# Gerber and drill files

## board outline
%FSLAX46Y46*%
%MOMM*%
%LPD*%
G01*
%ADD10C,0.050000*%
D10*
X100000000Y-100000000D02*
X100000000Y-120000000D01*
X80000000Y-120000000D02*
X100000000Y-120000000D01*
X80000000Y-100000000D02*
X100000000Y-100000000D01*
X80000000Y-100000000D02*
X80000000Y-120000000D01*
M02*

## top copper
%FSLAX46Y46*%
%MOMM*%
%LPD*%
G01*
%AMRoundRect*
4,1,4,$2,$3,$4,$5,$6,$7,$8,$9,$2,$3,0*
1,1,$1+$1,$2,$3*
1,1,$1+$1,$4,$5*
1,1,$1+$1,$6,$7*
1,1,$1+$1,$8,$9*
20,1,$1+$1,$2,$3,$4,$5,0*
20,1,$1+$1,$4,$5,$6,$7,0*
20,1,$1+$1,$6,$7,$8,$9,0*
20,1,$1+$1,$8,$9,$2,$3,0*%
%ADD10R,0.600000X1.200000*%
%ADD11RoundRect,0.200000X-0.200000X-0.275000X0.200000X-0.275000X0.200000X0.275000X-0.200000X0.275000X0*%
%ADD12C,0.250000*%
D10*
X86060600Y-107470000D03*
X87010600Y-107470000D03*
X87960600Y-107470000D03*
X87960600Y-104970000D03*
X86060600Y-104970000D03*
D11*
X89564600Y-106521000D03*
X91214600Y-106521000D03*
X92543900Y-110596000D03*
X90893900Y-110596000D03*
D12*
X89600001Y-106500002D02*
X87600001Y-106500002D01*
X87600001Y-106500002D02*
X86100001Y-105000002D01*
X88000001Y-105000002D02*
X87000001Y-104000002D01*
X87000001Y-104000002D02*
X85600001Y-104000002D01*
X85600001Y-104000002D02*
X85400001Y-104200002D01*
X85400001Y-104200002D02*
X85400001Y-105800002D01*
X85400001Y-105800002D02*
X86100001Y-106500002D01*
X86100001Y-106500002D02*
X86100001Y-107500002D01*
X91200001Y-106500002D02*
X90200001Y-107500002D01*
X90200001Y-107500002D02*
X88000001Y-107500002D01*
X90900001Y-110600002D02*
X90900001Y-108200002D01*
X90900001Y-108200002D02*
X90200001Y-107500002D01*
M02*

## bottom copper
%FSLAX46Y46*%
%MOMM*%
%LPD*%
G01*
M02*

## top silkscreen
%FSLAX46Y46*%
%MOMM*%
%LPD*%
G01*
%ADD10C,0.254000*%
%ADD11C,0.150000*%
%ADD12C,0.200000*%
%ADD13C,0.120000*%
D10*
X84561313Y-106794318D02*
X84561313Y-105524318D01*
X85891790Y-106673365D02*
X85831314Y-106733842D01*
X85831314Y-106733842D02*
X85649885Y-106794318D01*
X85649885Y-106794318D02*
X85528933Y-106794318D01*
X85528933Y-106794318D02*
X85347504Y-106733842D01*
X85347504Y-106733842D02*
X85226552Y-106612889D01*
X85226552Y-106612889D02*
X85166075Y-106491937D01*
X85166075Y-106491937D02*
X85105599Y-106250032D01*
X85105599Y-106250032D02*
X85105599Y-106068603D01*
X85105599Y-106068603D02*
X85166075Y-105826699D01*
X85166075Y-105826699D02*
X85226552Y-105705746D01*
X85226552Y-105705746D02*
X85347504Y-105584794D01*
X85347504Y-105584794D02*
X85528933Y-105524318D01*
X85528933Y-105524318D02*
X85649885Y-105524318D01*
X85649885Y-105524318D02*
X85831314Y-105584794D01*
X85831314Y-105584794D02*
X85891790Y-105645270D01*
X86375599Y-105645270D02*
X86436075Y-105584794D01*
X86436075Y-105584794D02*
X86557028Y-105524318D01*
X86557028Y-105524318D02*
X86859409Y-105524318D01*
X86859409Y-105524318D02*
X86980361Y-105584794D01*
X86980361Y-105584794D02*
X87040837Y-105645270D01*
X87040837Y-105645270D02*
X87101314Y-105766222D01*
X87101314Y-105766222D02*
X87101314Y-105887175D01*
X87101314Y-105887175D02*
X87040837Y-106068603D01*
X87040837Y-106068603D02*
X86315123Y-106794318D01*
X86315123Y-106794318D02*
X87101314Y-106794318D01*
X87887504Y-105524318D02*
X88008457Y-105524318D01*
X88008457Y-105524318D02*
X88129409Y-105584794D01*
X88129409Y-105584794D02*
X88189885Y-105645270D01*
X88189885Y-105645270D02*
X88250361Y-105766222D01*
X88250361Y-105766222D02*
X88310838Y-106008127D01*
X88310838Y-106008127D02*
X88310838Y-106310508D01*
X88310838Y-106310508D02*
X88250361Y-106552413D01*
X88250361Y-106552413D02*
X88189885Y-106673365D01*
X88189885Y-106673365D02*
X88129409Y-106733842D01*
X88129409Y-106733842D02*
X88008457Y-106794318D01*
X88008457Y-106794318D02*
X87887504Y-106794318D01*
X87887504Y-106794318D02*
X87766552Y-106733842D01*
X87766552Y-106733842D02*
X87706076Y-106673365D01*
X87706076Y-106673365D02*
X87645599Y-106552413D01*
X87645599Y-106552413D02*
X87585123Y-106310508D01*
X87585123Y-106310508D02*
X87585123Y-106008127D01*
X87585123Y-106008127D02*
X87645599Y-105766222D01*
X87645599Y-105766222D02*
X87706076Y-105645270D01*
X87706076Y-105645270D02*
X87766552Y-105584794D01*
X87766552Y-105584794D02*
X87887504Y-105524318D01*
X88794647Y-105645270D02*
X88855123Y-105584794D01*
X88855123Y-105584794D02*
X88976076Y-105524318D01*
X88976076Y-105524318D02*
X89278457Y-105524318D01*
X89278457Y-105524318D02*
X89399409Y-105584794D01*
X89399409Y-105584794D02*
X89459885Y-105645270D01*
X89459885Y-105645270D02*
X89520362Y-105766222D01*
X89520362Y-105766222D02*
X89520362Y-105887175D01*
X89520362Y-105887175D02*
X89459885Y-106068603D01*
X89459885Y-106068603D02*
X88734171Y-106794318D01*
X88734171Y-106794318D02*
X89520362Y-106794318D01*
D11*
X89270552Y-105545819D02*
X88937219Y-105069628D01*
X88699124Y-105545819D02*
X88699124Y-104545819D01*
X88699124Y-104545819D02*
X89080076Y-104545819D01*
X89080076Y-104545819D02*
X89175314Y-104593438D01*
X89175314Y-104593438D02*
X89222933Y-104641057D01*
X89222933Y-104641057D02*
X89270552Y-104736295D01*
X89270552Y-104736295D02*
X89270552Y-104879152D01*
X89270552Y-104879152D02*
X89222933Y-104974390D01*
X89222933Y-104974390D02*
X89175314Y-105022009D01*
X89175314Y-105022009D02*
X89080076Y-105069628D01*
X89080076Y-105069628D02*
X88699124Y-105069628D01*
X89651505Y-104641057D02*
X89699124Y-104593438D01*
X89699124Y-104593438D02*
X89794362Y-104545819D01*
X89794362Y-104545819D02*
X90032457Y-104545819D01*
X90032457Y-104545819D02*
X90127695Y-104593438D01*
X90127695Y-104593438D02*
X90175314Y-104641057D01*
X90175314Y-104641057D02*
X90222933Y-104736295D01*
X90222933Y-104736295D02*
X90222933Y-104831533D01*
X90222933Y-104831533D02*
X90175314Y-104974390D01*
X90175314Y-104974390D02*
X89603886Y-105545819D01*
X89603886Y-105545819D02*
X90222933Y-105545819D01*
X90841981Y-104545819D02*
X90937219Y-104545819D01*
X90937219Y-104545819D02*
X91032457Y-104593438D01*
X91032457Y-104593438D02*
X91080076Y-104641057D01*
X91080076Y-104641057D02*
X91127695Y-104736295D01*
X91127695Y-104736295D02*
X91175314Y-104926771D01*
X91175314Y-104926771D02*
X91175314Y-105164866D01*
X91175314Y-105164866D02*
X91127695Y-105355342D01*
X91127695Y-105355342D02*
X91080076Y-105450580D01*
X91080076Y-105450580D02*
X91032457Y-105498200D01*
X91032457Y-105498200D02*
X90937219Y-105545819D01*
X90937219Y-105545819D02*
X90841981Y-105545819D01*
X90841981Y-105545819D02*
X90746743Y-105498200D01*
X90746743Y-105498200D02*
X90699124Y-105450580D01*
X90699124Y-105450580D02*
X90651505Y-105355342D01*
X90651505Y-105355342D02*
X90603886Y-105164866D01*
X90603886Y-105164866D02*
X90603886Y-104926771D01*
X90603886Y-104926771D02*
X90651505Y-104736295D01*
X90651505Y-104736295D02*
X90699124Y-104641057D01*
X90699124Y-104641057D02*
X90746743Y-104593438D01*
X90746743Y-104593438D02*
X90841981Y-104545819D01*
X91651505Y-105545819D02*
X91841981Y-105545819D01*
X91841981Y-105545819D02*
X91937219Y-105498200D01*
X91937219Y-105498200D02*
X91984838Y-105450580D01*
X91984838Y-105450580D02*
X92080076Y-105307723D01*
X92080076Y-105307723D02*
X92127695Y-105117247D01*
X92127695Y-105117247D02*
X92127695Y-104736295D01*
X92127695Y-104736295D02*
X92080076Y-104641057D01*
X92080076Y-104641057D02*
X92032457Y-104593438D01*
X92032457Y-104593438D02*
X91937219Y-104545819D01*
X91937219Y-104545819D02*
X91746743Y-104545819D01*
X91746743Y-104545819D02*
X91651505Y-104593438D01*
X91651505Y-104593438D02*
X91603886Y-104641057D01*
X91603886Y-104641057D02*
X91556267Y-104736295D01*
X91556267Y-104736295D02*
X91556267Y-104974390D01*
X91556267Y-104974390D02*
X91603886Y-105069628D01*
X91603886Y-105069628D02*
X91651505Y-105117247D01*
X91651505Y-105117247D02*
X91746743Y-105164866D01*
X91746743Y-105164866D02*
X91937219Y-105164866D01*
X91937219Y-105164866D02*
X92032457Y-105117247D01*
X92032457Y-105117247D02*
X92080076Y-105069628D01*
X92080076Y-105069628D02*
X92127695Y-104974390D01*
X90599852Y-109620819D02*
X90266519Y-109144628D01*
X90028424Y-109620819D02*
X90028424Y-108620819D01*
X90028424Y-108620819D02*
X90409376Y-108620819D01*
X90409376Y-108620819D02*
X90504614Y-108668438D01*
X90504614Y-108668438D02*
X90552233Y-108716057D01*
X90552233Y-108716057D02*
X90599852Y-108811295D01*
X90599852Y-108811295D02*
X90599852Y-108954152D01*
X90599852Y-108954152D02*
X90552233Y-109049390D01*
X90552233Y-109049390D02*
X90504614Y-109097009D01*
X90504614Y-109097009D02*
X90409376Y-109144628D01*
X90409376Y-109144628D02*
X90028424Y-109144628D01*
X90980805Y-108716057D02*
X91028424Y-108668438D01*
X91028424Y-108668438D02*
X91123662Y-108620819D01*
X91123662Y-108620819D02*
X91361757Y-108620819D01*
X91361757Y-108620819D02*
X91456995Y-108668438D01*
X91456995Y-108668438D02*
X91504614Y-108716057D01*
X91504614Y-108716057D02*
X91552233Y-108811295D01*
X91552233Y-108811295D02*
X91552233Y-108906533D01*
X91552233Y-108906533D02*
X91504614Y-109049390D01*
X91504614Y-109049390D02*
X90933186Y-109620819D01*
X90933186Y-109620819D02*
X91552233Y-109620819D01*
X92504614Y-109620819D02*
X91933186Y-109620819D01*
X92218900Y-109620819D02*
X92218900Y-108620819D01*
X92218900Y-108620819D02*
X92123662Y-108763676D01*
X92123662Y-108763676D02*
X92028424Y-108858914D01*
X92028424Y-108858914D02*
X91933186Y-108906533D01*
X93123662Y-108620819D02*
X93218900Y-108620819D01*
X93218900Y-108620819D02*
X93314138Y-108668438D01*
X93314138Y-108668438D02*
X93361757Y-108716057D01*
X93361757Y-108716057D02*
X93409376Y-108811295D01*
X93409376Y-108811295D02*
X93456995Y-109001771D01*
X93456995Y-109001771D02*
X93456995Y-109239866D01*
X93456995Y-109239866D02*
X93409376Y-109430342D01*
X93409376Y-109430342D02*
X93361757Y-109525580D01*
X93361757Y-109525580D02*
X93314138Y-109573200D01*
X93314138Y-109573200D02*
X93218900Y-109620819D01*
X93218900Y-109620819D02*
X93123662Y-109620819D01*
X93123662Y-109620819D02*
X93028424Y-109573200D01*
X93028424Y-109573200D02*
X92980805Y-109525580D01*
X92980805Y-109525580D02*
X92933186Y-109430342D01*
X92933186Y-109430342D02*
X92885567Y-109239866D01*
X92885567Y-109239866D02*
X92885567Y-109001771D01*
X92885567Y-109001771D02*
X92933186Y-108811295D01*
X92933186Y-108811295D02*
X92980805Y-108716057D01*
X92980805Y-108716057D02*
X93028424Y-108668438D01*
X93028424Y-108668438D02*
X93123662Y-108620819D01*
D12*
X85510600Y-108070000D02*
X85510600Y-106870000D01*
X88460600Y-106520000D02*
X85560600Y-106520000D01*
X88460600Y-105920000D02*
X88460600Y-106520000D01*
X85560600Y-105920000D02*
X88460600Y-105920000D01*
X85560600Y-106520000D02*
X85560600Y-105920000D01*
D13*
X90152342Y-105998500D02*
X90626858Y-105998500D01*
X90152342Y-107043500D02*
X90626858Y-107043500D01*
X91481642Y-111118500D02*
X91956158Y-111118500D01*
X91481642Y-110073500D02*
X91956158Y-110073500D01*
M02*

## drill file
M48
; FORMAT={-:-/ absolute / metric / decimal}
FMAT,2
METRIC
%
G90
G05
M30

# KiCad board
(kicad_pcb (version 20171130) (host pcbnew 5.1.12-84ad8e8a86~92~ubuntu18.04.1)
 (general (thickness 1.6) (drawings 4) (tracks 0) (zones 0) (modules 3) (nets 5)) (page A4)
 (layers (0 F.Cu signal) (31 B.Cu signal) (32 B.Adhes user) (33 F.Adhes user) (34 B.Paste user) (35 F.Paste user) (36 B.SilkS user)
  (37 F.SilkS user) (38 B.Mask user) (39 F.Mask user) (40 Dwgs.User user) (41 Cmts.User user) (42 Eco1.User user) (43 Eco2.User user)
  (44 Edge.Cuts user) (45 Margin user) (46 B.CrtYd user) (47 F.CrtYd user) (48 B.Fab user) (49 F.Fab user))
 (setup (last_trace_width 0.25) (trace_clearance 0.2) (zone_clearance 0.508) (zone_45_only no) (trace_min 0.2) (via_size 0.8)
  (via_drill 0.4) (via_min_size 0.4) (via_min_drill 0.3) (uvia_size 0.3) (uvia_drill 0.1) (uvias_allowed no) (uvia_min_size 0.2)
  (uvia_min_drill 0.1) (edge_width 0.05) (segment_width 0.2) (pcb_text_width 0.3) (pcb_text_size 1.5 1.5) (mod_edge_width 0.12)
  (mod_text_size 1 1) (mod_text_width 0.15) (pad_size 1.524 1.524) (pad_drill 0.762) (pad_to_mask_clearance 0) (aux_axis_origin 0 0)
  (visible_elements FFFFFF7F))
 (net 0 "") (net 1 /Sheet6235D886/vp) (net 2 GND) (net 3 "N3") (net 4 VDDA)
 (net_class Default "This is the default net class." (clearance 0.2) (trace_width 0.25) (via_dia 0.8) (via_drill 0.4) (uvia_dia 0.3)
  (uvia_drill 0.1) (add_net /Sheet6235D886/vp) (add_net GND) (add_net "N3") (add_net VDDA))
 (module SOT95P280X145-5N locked (layer F.Cu) (at 87.010600 106.220000 90.000000)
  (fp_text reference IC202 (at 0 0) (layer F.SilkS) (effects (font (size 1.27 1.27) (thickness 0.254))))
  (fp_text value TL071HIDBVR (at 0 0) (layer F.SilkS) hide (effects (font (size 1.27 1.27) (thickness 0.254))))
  (fp_line (start -1.85 -1.5) (end -0.65 -1.5) (layer F.SilkS) (width 0.2))
  (fp_line (start -0.3 1.45) (end -0.3 -1.45) (layer F.SilkS) (width 0.2))
  (fp_line (start 0.3 1.45) (end -0.3 1.45) (layer F.SilkS) (width 0.2))
  (fp_line (start 0.3 -1.45) (end 0.3 1.45) (layer F.SilkS) (width 0.2))
  (fp_line (start -0.3 -1.45) (end 0.3 -1.45) (layer F.SilkS) (width 0.2))
  (pad 1 smd rect (at -1.25 -0.95 180.000000) (size 0.6 1.2) (layers F.Cu F.Mask F.Paste) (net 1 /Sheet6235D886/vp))
  (pad 2 smd rect (at -1.25 0 180.000000) (size 0.6 1.2) (layers F.Cu F.Mask F.Paste) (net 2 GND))
  (pad 3 smd rect (at -1.25 0.95 180.000000) (size 0.6 1.2) (layers F.Cu F.Mask F.Paste) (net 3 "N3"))
  (pad 4 smd rect (at 1.25 0.95 180.000000) (size 0.6 1.2) (layers F.Cu F.Mask F.Paste) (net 1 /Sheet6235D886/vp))
  (pad 5 smd rect (at 1.25 -0.95 180.000000) (size 0.6 1.2) (layers F.Cu F.Mask F.Paste) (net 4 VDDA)))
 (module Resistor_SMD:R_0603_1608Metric (layer F.Cu) (at 90.389600 106.521000)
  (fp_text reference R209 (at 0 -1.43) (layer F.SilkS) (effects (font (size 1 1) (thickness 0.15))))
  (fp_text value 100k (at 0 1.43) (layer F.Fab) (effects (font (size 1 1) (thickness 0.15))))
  (fp_line (start -0.237258 -0.5225) (end 0.237258 -0.5225) (layer F.SilkS) (width 0.12))
  (fp_line (start -0.237258 0.5225) (end 0.237258 0.5225) (layer F.SilkS) (width 0.12))
  (pad 1 smd roundrect (at -0.825 0) (size 0.8 0.95) (layers F.Cu F.Mask F.Paste) (roundrect_rratio 0.25) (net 4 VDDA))
  (pad 2 smd roundrect (at 0.825 0) (size 0.8 0.95) (layers F.Cu F.Mask F.Paste) (roundrect_rratio 0.25) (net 3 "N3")))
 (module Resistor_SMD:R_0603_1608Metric (layer F.Cu) (at 91.718900 110.596000)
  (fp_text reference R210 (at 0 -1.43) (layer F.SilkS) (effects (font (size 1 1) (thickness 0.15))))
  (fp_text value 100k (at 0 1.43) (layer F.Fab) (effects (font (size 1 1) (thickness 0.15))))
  (fp_line (start -0.237258 0.5225) (end 0.237258 0.5225) (layer F.SilkS) (width 0.12))
  (fp_line (start -0.237258 -0.5225) (end 0.237258 -0.5225) (layer F.SilkS) (width 0.12))
  (pad 2 smd roundrect (at 0.825 0) (size 0.8 0.95) (layers F.Cu F.Mask F.Paste) (roundrect_rratio 0.25) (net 2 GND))
  (pad 1 smd roundrect (at -0.825 0) (size 0.8 0.95) (layers F.Cu F.Mask F.Paste) (roundrect_rratio 0.25) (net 3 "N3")))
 (gr_line (start 100 100) (end 100 120) (layer Edge.Cuts) (width 0.05))
 (gr_line (start 80 120) (end 100 120) (layer Edge.Cuts) (width 0.05))
 (gr_line (start 80 100) (end 100 100) (layer Edge.Cuts) (width 0.05))
 (gr_line (start 80 100) (end 80 120) (layer Edge.Cuts) (width 0.05))
 (segment (start 89.600001 106.500002) (end 87.600001 106.500002) (width 0.250000) (layer F.Cu) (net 4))
 (segment (start 87.600001 106.500002) (end 86.100001 105.000002) (width 0.250000) (layer F.Cu) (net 4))
 (segment (start 88.000001 105.000002) (end 87.000001 104.000002) (width 0.250000) (layer F.Cu) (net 1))
 (segment (start 87.000001 104.000002) (end 85.600001 104.000002) (width 0.250000) (layer F.Cu) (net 1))
 (segment (start 85.600001 104.000002) (end 85.400001 104.200002) (width 0.250000) (layer F.Cu) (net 1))
 (segment (start 85.400001 104.200002) (end 85.400001 105.800002) (width 0.250000) (layer F.Cu) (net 1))
 (segment (start 85.400001 105.800002) (end 86.100001 106.500002) (width 0.250000) (layer F.Cu) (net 1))
 (segment (start 86.100001 106.500002) (end 86.100001 107.500002) (width 0.250000) (layer F.Cu) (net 1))
 (segment (start 91.200001 106.500002) (end 90.200001 107.500002) (width 0.250000) (layer F.Cu) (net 3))
 (segment (start 90.200001 107.500002) (end 88.000001 107.500002) (width 0.250000) (layer F.Cu) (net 3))
 (segment (start 90.900001 110.600002) (end 90.900001 108.200002) (width 0.250000) (layer F.Cu) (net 3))
 (segment (start 90.900001 108.200002) (end 90.200001 107.500002) (width 0.250000) (layer F.Cu) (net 3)))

